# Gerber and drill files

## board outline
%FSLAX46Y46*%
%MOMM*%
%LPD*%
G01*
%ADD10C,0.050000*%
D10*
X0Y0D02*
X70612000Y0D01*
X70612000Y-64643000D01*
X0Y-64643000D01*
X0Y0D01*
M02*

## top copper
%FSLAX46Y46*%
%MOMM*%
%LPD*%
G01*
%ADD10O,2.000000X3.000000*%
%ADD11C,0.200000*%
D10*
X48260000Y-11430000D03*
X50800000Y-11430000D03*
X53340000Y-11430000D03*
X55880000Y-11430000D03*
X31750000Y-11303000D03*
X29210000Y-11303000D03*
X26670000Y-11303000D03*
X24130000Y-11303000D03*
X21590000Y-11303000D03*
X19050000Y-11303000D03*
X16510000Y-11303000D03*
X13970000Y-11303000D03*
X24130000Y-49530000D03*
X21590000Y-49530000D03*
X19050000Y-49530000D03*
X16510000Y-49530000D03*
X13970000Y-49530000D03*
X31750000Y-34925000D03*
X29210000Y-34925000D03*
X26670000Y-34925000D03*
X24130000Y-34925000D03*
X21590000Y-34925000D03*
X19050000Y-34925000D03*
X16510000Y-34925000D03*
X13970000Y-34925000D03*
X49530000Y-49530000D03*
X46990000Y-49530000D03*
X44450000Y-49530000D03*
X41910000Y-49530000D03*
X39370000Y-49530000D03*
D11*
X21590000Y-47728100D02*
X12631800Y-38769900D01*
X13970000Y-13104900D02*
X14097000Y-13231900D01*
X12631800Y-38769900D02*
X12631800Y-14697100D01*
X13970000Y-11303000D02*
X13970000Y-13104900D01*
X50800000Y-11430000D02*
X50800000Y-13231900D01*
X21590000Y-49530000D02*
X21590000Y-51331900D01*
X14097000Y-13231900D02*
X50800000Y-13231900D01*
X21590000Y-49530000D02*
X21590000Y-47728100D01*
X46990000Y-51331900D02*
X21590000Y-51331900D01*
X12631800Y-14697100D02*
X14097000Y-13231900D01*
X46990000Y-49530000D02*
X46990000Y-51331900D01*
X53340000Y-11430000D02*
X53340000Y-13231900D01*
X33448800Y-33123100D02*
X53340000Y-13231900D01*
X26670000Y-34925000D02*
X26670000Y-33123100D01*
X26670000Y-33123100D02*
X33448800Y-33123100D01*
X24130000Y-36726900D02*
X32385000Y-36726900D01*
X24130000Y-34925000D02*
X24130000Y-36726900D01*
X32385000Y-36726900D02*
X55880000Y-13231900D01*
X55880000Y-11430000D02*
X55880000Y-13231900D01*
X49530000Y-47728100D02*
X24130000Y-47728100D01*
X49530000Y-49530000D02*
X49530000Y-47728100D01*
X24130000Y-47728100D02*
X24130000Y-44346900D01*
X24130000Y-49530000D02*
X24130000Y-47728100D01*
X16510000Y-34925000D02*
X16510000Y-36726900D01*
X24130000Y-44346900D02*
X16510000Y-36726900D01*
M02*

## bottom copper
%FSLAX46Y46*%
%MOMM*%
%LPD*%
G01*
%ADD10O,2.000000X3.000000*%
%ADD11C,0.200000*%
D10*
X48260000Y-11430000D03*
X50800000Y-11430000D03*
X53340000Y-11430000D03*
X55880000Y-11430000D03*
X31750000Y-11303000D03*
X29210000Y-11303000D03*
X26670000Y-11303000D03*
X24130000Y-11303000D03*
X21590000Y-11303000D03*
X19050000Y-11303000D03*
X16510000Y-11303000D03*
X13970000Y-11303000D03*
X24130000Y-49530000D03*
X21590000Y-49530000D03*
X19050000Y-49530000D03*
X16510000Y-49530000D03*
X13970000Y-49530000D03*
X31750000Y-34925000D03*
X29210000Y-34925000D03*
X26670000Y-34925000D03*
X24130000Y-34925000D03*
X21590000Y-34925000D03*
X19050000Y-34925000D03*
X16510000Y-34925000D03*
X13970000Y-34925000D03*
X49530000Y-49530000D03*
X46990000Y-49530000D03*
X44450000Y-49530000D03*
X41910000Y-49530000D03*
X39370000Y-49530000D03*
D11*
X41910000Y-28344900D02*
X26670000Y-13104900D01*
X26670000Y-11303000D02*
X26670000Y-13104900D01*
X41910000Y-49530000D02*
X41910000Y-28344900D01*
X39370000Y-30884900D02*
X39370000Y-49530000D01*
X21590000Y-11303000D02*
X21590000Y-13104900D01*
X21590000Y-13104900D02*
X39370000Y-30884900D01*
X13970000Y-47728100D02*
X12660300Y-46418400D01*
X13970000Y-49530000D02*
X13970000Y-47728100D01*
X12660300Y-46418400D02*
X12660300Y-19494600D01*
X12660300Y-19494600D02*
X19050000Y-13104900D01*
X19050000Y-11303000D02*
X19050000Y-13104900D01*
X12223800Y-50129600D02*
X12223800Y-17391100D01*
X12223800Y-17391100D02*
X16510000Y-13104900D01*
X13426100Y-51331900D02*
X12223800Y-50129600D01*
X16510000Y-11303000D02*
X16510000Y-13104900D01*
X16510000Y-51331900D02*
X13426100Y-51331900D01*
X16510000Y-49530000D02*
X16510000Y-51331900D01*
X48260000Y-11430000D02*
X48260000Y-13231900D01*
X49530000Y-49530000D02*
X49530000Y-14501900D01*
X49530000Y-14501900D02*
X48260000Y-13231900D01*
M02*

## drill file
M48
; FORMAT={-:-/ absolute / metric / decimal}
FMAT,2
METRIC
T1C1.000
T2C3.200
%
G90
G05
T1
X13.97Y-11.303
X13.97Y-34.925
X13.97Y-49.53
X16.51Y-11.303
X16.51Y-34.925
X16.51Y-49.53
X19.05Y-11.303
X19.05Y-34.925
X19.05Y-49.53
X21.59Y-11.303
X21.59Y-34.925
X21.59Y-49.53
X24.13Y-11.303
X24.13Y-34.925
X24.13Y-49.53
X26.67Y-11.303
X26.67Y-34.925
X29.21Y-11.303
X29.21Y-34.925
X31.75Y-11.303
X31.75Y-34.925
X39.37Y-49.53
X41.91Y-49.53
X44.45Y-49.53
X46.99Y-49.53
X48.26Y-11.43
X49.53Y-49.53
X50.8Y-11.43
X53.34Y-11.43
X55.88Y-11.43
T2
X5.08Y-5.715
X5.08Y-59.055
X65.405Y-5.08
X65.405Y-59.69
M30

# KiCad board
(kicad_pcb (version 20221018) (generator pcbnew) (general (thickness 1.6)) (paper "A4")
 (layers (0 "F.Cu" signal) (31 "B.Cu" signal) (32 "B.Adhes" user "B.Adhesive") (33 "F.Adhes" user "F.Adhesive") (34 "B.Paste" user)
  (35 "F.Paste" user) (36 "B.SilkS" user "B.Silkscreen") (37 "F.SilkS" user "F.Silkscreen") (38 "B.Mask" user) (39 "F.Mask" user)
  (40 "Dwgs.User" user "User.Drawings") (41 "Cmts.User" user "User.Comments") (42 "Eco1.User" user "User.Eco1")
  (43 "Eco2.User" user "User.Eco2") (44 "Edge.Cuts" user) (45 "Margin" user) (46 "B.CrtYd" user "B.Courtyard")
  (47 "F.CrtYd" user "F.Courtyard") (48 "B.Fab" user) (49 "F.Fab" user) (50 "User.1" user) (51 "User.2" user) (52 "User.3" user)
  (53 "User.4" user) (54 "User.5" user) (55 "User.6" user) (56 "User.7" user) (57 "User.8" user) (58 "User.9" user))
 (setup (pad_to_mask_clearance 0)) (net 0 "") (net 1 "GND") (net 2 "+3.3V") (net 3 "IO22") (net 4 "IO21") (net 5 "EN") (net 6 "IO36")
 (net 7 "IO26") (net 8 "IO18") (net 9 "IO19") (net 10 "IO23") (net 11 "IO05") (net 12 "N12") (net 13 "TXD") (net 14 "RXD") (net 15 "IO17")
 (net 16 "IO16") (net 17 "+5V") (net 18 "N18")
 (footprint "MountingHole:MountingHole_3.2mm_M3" (layer "F.Cu") (at 65.405 59.69)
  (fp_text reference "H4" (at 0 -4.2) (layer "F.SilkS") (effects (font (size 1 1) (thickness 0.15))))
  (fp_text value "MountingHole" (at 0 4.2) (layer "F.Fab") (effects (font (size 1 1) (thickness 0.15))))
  (pad "" np_thru_hole circle (at 0 0) (size 3.2 3.2) (drill 3.2) (layers "*.Cu" "*.Mask")))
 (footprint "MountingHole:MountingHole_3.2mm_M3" (layer "F.Cu") (at 65.405 5.08)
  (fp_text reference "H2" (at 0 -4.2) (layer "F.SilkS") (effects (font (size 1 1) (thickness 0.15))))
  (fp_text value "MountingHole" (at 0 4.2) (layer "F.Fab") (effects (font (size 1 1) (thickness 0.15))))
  (pad "" np_thru_hole circle (at 0 0) (size 3.2 3.2) (drill 3.2) (layers "*.Cu" "*.Mask")))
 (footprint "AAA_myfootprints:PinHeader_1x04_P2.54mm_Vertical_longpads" (layer "F.Cu") (at 48.26 11.43 90)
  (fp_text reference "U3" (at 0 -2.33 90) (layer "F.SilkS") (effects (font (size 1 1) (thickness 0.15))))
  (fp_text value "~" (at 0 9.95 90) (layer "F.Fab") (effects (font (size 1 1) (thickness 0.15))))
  (pad "1" thru_hole oval (at 0 0 90) (size 3 2) (drill 1) (layers "*.Cu" "*.Mask") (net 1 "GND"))
  (pad "2" thru_hole oval (at 0 2.54 90) (size 3 2) (drill 1) (layers "*.Cu" "*.Mask") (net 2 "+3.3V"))
  (pad "3" thru_hole oval (at 0 5.08 90) (size 3 2) (drill 1) (layers "*.Cu" "*.Mask") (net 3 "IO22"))
  (pad "4" thru_hole oval (at 0 7.62 90) (size 3 2) (drill 1) (layers "*.Cu" "*.Mask") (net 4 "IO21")))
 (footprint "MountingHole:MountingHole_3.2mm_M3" (layer "F.Cu") (at 5.08 5.715)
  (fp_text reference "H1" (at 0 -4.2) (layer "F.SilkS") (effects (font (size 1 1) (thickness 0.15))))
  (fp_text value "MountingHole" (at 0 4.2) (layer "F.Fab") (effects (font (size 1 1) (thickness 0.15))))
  (pad "" np_thru_hole circle (at 0 0) (size 3.2 3.2) (drill 3.2) (layers "*.Cu" "*.Mask")))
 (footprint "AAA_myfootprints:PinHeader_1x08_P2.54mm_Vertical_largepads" (layer "F.Cu") (at 31.75 11.303 -90)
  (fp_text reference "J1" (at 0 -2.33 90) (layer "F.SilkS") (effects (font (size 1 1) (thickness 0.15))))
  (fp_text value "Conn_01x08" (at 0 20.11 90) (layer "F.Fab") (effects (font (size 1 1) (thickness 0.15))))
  (pad "1" thru_hole oval (at 0 0 270) (size 3 2) (drill 1) (layers "*.Cu" "*.Mask") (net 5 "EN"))
  (pad "2" thru_hole oval (at 0 2.54 270) (size 3 2) (drill 1) (layers "*.Cu" "*.Mask") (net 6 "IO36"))
  (pad "3" thru_hole oval (at 0 5.08 270) (size 3 2) (drill 1) (layers "*.Cu" "*.Mask") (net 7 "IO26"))
  (pad "4" thru_hole oval (at 0 7.62 270) (size 3 2) (drill 1) (layers "*.Cu" "*.Mask") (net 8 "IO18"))
  (pad "5" thru_hole oval (at 0 10.16 270) (size 3 2) (drill 1) (layers "*.Cu" "*.Mask") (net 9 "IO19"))
  (pad "6" thru_hole oval (at 0 12.7 270) (size 3 2) (drill 1) (layers "*.Cu" "*.Mask") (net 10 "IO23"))
  (pad "7" thru_hole oval (at 0 15.24 270) (size 3 2) (drill 1) (layers "*.Cu" "*.Mask") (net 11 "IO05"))
  (pad "8" thru_hole oval (at 0 17.78 270) (size 3 2) (drill 1) (layers "*.Cu" "*.Mask") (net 2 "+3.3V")))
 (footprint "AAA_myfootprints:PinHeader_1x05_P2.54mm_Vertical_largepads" (layer "F.Cu") (at 24.13 49.53 -90)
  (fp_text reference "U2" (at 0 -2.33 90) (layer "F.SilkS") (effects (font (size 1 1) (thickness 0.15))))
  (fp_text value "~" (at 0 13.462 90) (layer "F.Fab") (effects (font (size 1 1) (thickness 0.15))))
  (pad "1" thru_hole oval (at 0 0 270) (size 3 2) (drill 1) (layers "*.Cu" "*.Mask") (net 1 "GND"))
  (pad "2" thru_hole oval (at 0 2.54 270) (size 3 2) (drill 1) (layers "*.Cu" "*.Mask") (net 2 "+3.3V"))
  (pad "3" thru_hole oval (at 0 5.08 270) (size 3 2) (drill 1) (layers "*.Cu" "*.Mask") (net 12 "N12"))
  (pad "4" thru_hole oval (at 0 7.62 270) (size 3 2) (drill 1) (layers "*.Cu" "*.Mask") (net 11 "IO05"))
  (pad "5" thru_hole oval (at 0 10.16 270) (size 3 2) (drill 1) (layers "*.Cu" "*.Mask") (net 10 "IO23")))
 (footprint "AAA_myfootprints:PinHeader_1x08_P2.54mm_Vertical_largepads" (layer "F.Cu") (at 31.75 34.925 -90)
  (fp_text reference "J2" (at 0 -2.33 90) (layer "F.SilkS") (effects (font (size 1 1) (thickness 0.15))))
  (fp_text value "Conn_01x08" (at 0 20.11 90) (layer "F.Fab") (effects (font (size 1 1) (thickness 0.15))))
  (pad "1" thru_hole oval (at 0 0 270) (size 3 2) (drill 1) (layers "*.Cu" "*.Mask") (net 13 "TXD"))
  (pad "2" thru_hole oval (at 0 2.54 270) (size 3 2) (drill 1) (layers "*.Cu" "*.Mask") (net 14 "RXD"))
  (pad "3" thru_hole oval (at 0 5.08 270) (size 3 2) (drill 1) (layers "*.Cu" "*.Mask") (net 3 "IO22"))
  (pad "4" thru_hole oval (at 0 7.62 270) (size 3 2) (drill 1) (layers "*.Cu" "*.Mask") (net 4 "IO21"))
  (pad "5" thru_hole oval (at 0 10.16 270) (size 3 2) (drill 1) (layers "*.Cu" "*.Mask") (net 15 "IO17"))
  (pad "6" thru_hole oval (at 0 12.7 270) (size 3 2) (drill 1) (layers "*.Cu" "*.Mask") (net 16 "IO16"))
  (pad "7" thru_hole oval (at 0 15.24 270) (size 3 2) (drill 1) (layers "*.Cu" "*.Mask") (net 1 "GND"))
  (pad "8" thru_hole oval (at 0 17.78 270) (size 3 2) (drill 1) (layers "*.Cu" "*.Mask") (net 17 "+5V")))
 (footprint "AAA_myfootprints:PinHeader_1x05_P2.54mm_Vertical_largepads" (layer "F.Cu") (at 49.53 49.53 -90)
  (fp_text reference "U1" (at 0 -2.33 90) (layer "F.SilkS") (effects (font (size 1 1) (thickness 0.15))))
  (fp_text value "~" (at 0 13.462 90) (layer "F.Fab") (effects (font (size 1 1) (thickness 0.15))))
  (pad "1" thru_hole oval (at 0 0 270) (size 3 2) (drill 1) (layers "*.Cu" "*.Mask") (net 1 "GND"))
  (pad "2" thru_hole oval (at 0 2.54 270) (size 3 2) (drill 1) (layers "*.Cu" "*.Mask") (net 2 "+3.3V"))
  (pad "3" thru_hole oval (at 0 5.08 270) (size 3 2) (drill 1) (layers "*.Cu" "*.Mask") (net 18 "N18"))
  (pad "4" thru_hole oval (at 0 7.62 270) (size 3 2) (drill 1) (layers "*.Cu" "*.Mask") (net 7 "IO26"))
  (pad "5" thru_hole oval (at 0 10.16 270) (size 3 2) (drill 1) (layers "*.Cu" "*.Mask") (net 9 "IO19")))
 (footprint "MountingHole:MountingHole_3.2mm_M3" (layer "F.Cu") (at 5.08 59.055)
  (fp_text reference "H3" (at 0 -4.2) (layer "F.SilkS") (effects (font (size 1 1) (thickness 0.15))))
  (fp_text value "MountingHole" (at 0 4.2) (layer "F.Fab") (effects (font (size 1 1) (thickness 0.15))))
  (pad "" np_thru_hole circle (at 0 0) (size 3.2 3.2) (drill 3.2) (layers "*.Cu" "*.Mask")))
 (gr_rect (start 0 0) (end 70.612 64.643) (stroke (width 0.05) (type default)) (fill none) (layer "Edge.Cuts"))
 (segment (start 41.91 28.3449) (end 26.67 13.1049) (width 0.2) (layer "B.Cu") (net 7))
 (segment (start 26.67 11.303) (end 26.67 13.1049) (width 0.2) (layer "B.Cu") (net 7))
 (segment (start 41.91 49.53) (end 41.91 28.3449) (width 0.2) (layer "B.Cu") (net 7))
 (segment (start 39.37 30.8849) (end 39.37 49.53) (width 0.2) (layer "B.Cu") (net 9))
 (segment (start 21.59 11.303) (end 21.59 13.1049) (width 0.2) (layer "B.Cu") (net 9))
 (segment (start 21.59 13.1049) (end 39.37 30.8849) (width 0.2) (layer "B.Cu") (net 9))
 (segment (start 13.97 47.7281) (end 12.6603 46.4184) (width 0.2) (layer "B.Cu") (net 10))
 (segment (start 13.97 49.53) (end 13.97 47.7281) (width 0.2) (layer "B.Cu") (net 10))
 (segment (start 12.6603 46.4184) (end 12.6603 19.4946) (width 0.2) (layer "B.Cu") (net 10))
 (segment (start 12.6603 19.4946) (end 19.05 13.1049) (width 0.2) (layer "B.Cu") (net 10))
 (segment (start 19.05 11.303) (end 19.05 13.1049) (width 0.2) (layer "B.Cu") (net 10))
 (segment (start 12.2238 50.1296) (end 12.2238 17.3911) (width 0.2) (layer "B.Cu") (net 11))
 (segment (start 12.2238 17.3911) (end 16.51 13.1049) (width 0.2) (layer "B.Cu") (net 11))
 (segment (start 13.4261 51.3319) (end 12.2238 50.1296) (width 0.2) (layer "B.Cu") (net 11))
 (segment (start 16.51 11.303) (end 16.51 13.1049) (width 0.2) (layer "B.Cu") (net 11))
 (segment (start 16.51 51.3319) (end 13.4261 51.3319) (width 0.2) (layer "B.Cu") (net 11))
 (segment (start 16.51 49.53) (end 16.51 51.3319) (width 0.2) (layer "B.Cu") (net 11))
 (segment (start 21.59 47.7281) (end 12.6318 38.7699) (width 0.2) (layer "F.Cu") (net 2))
 (segment (start 13.97 13.1049) (end 14.097 13.2319) (width 0.2) (layer "F.Cu") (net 2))
 (segment (start 12.6318 38.7699) (end 12.6318 14.6971) (width 0.2) (layer "F.Cu") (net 2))
 (segment (start 13.97 11.303) (end 13.97 13.1049) (width 0.2) (layer "F.Cu") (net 2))
 (segment (start 50.8 11.43) (end 50.8 13.2319) (width 0.2) (layer "F.Cu") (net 2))
 (segment (start 21.59 49.53) (end 21.59 51.3319) (width 0.2) (layer "F.Cu") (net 2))
 (segment (start 14.097 13.2319) (end 50.8 13.2319) (width 0.2) (layer "F.Cu") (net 2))
 (segment (start 21.59 49.53) (end 21.59 47.7281) (width 0.2) (layer "F.Cu") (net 2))
 (segment (start 46.99 51.3319) (end 21.59 51.3319) (width 0.2) (layer "F.Cu") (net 2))
 (segment (start 12.6318 14.6971) (end 14.097 13.2319) (width 0.2) (layer "F.Cu") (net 2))
 (segment (start 46.99 49.53) (end 46.99 51.3319) (width 0.2) (layer "F.Cu") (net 2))
 (segment (start 53.34 11.43) (end 53.34 13.2319) (width 0.2) (layer "F.Cu") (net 3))
 (segment (start 33.4488 33.1231) (end 53.34 13.2319) (width 0.2) (layer "F.Cu") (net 3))
 (segment (start 26.67 34.925) (end 26.67 33.1231) (width 0.2) (layer "F.Cu") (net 3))
 (segment (start 26.67 33.1231) (end 33.4488 33.1231) (width 0.2) (layer "F.Cu") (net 3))
 (segment (start 24.13 36.7269) (end 32.385 36.7269) (width 0.2) (layer "F.Cu") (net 4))
 (segment (start 24.13 34.925) (end 24.13 36.7269) (width 0.2) (layer "F.Cu") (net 4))
 (segment (start 32.385 36.7269) (end 55.88 13.2319) (width 0.2) (layer "F.Cu") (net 4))
 (segment (start 55.88 11.43) (end 55.88 13.2319) (width 0.2) (layer "F.Cu") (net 4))
 (segment (start 49.53 47.7281) (end 24.13 47.7281) (width 0.2) (layer "F.Cu") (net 1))
 (segment (start 49.53 49.53) (end 49.53 47.7281) (width 0.2) (layer "F.Cu") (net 1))
 (segment (start 24.13 47.7281) (end 24.13 44.3469) (width 0.2) (layer "F.Cu") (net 1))
 (segment (start 24.13 49.53) (end 24.13 47.7281) (width 0.2) (layer "F.Cu") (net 1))
 (segment (start 16.51 34.925) (end 16.51 36.7269) (width 0.2) (layer "F.Cu") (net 1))
 (segment (start 24.13 44.3469) (end 16.51 36.7269) (width 0.2) (layer "F.Cu") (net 1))
 (segment (start 48.26 11.43) (end 48.26 13.2319) (width 0.2) (layer "B.Cu") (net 1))
 (segment (start 49.53 49.53) (end 49.53 14.5019) (width 0.2) (layer "B.Cu") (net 1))
 (segment (start 49.53 14.5019) (end 48.26 13.2319) (width 0.2) (layer "B.Cu") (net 1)))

